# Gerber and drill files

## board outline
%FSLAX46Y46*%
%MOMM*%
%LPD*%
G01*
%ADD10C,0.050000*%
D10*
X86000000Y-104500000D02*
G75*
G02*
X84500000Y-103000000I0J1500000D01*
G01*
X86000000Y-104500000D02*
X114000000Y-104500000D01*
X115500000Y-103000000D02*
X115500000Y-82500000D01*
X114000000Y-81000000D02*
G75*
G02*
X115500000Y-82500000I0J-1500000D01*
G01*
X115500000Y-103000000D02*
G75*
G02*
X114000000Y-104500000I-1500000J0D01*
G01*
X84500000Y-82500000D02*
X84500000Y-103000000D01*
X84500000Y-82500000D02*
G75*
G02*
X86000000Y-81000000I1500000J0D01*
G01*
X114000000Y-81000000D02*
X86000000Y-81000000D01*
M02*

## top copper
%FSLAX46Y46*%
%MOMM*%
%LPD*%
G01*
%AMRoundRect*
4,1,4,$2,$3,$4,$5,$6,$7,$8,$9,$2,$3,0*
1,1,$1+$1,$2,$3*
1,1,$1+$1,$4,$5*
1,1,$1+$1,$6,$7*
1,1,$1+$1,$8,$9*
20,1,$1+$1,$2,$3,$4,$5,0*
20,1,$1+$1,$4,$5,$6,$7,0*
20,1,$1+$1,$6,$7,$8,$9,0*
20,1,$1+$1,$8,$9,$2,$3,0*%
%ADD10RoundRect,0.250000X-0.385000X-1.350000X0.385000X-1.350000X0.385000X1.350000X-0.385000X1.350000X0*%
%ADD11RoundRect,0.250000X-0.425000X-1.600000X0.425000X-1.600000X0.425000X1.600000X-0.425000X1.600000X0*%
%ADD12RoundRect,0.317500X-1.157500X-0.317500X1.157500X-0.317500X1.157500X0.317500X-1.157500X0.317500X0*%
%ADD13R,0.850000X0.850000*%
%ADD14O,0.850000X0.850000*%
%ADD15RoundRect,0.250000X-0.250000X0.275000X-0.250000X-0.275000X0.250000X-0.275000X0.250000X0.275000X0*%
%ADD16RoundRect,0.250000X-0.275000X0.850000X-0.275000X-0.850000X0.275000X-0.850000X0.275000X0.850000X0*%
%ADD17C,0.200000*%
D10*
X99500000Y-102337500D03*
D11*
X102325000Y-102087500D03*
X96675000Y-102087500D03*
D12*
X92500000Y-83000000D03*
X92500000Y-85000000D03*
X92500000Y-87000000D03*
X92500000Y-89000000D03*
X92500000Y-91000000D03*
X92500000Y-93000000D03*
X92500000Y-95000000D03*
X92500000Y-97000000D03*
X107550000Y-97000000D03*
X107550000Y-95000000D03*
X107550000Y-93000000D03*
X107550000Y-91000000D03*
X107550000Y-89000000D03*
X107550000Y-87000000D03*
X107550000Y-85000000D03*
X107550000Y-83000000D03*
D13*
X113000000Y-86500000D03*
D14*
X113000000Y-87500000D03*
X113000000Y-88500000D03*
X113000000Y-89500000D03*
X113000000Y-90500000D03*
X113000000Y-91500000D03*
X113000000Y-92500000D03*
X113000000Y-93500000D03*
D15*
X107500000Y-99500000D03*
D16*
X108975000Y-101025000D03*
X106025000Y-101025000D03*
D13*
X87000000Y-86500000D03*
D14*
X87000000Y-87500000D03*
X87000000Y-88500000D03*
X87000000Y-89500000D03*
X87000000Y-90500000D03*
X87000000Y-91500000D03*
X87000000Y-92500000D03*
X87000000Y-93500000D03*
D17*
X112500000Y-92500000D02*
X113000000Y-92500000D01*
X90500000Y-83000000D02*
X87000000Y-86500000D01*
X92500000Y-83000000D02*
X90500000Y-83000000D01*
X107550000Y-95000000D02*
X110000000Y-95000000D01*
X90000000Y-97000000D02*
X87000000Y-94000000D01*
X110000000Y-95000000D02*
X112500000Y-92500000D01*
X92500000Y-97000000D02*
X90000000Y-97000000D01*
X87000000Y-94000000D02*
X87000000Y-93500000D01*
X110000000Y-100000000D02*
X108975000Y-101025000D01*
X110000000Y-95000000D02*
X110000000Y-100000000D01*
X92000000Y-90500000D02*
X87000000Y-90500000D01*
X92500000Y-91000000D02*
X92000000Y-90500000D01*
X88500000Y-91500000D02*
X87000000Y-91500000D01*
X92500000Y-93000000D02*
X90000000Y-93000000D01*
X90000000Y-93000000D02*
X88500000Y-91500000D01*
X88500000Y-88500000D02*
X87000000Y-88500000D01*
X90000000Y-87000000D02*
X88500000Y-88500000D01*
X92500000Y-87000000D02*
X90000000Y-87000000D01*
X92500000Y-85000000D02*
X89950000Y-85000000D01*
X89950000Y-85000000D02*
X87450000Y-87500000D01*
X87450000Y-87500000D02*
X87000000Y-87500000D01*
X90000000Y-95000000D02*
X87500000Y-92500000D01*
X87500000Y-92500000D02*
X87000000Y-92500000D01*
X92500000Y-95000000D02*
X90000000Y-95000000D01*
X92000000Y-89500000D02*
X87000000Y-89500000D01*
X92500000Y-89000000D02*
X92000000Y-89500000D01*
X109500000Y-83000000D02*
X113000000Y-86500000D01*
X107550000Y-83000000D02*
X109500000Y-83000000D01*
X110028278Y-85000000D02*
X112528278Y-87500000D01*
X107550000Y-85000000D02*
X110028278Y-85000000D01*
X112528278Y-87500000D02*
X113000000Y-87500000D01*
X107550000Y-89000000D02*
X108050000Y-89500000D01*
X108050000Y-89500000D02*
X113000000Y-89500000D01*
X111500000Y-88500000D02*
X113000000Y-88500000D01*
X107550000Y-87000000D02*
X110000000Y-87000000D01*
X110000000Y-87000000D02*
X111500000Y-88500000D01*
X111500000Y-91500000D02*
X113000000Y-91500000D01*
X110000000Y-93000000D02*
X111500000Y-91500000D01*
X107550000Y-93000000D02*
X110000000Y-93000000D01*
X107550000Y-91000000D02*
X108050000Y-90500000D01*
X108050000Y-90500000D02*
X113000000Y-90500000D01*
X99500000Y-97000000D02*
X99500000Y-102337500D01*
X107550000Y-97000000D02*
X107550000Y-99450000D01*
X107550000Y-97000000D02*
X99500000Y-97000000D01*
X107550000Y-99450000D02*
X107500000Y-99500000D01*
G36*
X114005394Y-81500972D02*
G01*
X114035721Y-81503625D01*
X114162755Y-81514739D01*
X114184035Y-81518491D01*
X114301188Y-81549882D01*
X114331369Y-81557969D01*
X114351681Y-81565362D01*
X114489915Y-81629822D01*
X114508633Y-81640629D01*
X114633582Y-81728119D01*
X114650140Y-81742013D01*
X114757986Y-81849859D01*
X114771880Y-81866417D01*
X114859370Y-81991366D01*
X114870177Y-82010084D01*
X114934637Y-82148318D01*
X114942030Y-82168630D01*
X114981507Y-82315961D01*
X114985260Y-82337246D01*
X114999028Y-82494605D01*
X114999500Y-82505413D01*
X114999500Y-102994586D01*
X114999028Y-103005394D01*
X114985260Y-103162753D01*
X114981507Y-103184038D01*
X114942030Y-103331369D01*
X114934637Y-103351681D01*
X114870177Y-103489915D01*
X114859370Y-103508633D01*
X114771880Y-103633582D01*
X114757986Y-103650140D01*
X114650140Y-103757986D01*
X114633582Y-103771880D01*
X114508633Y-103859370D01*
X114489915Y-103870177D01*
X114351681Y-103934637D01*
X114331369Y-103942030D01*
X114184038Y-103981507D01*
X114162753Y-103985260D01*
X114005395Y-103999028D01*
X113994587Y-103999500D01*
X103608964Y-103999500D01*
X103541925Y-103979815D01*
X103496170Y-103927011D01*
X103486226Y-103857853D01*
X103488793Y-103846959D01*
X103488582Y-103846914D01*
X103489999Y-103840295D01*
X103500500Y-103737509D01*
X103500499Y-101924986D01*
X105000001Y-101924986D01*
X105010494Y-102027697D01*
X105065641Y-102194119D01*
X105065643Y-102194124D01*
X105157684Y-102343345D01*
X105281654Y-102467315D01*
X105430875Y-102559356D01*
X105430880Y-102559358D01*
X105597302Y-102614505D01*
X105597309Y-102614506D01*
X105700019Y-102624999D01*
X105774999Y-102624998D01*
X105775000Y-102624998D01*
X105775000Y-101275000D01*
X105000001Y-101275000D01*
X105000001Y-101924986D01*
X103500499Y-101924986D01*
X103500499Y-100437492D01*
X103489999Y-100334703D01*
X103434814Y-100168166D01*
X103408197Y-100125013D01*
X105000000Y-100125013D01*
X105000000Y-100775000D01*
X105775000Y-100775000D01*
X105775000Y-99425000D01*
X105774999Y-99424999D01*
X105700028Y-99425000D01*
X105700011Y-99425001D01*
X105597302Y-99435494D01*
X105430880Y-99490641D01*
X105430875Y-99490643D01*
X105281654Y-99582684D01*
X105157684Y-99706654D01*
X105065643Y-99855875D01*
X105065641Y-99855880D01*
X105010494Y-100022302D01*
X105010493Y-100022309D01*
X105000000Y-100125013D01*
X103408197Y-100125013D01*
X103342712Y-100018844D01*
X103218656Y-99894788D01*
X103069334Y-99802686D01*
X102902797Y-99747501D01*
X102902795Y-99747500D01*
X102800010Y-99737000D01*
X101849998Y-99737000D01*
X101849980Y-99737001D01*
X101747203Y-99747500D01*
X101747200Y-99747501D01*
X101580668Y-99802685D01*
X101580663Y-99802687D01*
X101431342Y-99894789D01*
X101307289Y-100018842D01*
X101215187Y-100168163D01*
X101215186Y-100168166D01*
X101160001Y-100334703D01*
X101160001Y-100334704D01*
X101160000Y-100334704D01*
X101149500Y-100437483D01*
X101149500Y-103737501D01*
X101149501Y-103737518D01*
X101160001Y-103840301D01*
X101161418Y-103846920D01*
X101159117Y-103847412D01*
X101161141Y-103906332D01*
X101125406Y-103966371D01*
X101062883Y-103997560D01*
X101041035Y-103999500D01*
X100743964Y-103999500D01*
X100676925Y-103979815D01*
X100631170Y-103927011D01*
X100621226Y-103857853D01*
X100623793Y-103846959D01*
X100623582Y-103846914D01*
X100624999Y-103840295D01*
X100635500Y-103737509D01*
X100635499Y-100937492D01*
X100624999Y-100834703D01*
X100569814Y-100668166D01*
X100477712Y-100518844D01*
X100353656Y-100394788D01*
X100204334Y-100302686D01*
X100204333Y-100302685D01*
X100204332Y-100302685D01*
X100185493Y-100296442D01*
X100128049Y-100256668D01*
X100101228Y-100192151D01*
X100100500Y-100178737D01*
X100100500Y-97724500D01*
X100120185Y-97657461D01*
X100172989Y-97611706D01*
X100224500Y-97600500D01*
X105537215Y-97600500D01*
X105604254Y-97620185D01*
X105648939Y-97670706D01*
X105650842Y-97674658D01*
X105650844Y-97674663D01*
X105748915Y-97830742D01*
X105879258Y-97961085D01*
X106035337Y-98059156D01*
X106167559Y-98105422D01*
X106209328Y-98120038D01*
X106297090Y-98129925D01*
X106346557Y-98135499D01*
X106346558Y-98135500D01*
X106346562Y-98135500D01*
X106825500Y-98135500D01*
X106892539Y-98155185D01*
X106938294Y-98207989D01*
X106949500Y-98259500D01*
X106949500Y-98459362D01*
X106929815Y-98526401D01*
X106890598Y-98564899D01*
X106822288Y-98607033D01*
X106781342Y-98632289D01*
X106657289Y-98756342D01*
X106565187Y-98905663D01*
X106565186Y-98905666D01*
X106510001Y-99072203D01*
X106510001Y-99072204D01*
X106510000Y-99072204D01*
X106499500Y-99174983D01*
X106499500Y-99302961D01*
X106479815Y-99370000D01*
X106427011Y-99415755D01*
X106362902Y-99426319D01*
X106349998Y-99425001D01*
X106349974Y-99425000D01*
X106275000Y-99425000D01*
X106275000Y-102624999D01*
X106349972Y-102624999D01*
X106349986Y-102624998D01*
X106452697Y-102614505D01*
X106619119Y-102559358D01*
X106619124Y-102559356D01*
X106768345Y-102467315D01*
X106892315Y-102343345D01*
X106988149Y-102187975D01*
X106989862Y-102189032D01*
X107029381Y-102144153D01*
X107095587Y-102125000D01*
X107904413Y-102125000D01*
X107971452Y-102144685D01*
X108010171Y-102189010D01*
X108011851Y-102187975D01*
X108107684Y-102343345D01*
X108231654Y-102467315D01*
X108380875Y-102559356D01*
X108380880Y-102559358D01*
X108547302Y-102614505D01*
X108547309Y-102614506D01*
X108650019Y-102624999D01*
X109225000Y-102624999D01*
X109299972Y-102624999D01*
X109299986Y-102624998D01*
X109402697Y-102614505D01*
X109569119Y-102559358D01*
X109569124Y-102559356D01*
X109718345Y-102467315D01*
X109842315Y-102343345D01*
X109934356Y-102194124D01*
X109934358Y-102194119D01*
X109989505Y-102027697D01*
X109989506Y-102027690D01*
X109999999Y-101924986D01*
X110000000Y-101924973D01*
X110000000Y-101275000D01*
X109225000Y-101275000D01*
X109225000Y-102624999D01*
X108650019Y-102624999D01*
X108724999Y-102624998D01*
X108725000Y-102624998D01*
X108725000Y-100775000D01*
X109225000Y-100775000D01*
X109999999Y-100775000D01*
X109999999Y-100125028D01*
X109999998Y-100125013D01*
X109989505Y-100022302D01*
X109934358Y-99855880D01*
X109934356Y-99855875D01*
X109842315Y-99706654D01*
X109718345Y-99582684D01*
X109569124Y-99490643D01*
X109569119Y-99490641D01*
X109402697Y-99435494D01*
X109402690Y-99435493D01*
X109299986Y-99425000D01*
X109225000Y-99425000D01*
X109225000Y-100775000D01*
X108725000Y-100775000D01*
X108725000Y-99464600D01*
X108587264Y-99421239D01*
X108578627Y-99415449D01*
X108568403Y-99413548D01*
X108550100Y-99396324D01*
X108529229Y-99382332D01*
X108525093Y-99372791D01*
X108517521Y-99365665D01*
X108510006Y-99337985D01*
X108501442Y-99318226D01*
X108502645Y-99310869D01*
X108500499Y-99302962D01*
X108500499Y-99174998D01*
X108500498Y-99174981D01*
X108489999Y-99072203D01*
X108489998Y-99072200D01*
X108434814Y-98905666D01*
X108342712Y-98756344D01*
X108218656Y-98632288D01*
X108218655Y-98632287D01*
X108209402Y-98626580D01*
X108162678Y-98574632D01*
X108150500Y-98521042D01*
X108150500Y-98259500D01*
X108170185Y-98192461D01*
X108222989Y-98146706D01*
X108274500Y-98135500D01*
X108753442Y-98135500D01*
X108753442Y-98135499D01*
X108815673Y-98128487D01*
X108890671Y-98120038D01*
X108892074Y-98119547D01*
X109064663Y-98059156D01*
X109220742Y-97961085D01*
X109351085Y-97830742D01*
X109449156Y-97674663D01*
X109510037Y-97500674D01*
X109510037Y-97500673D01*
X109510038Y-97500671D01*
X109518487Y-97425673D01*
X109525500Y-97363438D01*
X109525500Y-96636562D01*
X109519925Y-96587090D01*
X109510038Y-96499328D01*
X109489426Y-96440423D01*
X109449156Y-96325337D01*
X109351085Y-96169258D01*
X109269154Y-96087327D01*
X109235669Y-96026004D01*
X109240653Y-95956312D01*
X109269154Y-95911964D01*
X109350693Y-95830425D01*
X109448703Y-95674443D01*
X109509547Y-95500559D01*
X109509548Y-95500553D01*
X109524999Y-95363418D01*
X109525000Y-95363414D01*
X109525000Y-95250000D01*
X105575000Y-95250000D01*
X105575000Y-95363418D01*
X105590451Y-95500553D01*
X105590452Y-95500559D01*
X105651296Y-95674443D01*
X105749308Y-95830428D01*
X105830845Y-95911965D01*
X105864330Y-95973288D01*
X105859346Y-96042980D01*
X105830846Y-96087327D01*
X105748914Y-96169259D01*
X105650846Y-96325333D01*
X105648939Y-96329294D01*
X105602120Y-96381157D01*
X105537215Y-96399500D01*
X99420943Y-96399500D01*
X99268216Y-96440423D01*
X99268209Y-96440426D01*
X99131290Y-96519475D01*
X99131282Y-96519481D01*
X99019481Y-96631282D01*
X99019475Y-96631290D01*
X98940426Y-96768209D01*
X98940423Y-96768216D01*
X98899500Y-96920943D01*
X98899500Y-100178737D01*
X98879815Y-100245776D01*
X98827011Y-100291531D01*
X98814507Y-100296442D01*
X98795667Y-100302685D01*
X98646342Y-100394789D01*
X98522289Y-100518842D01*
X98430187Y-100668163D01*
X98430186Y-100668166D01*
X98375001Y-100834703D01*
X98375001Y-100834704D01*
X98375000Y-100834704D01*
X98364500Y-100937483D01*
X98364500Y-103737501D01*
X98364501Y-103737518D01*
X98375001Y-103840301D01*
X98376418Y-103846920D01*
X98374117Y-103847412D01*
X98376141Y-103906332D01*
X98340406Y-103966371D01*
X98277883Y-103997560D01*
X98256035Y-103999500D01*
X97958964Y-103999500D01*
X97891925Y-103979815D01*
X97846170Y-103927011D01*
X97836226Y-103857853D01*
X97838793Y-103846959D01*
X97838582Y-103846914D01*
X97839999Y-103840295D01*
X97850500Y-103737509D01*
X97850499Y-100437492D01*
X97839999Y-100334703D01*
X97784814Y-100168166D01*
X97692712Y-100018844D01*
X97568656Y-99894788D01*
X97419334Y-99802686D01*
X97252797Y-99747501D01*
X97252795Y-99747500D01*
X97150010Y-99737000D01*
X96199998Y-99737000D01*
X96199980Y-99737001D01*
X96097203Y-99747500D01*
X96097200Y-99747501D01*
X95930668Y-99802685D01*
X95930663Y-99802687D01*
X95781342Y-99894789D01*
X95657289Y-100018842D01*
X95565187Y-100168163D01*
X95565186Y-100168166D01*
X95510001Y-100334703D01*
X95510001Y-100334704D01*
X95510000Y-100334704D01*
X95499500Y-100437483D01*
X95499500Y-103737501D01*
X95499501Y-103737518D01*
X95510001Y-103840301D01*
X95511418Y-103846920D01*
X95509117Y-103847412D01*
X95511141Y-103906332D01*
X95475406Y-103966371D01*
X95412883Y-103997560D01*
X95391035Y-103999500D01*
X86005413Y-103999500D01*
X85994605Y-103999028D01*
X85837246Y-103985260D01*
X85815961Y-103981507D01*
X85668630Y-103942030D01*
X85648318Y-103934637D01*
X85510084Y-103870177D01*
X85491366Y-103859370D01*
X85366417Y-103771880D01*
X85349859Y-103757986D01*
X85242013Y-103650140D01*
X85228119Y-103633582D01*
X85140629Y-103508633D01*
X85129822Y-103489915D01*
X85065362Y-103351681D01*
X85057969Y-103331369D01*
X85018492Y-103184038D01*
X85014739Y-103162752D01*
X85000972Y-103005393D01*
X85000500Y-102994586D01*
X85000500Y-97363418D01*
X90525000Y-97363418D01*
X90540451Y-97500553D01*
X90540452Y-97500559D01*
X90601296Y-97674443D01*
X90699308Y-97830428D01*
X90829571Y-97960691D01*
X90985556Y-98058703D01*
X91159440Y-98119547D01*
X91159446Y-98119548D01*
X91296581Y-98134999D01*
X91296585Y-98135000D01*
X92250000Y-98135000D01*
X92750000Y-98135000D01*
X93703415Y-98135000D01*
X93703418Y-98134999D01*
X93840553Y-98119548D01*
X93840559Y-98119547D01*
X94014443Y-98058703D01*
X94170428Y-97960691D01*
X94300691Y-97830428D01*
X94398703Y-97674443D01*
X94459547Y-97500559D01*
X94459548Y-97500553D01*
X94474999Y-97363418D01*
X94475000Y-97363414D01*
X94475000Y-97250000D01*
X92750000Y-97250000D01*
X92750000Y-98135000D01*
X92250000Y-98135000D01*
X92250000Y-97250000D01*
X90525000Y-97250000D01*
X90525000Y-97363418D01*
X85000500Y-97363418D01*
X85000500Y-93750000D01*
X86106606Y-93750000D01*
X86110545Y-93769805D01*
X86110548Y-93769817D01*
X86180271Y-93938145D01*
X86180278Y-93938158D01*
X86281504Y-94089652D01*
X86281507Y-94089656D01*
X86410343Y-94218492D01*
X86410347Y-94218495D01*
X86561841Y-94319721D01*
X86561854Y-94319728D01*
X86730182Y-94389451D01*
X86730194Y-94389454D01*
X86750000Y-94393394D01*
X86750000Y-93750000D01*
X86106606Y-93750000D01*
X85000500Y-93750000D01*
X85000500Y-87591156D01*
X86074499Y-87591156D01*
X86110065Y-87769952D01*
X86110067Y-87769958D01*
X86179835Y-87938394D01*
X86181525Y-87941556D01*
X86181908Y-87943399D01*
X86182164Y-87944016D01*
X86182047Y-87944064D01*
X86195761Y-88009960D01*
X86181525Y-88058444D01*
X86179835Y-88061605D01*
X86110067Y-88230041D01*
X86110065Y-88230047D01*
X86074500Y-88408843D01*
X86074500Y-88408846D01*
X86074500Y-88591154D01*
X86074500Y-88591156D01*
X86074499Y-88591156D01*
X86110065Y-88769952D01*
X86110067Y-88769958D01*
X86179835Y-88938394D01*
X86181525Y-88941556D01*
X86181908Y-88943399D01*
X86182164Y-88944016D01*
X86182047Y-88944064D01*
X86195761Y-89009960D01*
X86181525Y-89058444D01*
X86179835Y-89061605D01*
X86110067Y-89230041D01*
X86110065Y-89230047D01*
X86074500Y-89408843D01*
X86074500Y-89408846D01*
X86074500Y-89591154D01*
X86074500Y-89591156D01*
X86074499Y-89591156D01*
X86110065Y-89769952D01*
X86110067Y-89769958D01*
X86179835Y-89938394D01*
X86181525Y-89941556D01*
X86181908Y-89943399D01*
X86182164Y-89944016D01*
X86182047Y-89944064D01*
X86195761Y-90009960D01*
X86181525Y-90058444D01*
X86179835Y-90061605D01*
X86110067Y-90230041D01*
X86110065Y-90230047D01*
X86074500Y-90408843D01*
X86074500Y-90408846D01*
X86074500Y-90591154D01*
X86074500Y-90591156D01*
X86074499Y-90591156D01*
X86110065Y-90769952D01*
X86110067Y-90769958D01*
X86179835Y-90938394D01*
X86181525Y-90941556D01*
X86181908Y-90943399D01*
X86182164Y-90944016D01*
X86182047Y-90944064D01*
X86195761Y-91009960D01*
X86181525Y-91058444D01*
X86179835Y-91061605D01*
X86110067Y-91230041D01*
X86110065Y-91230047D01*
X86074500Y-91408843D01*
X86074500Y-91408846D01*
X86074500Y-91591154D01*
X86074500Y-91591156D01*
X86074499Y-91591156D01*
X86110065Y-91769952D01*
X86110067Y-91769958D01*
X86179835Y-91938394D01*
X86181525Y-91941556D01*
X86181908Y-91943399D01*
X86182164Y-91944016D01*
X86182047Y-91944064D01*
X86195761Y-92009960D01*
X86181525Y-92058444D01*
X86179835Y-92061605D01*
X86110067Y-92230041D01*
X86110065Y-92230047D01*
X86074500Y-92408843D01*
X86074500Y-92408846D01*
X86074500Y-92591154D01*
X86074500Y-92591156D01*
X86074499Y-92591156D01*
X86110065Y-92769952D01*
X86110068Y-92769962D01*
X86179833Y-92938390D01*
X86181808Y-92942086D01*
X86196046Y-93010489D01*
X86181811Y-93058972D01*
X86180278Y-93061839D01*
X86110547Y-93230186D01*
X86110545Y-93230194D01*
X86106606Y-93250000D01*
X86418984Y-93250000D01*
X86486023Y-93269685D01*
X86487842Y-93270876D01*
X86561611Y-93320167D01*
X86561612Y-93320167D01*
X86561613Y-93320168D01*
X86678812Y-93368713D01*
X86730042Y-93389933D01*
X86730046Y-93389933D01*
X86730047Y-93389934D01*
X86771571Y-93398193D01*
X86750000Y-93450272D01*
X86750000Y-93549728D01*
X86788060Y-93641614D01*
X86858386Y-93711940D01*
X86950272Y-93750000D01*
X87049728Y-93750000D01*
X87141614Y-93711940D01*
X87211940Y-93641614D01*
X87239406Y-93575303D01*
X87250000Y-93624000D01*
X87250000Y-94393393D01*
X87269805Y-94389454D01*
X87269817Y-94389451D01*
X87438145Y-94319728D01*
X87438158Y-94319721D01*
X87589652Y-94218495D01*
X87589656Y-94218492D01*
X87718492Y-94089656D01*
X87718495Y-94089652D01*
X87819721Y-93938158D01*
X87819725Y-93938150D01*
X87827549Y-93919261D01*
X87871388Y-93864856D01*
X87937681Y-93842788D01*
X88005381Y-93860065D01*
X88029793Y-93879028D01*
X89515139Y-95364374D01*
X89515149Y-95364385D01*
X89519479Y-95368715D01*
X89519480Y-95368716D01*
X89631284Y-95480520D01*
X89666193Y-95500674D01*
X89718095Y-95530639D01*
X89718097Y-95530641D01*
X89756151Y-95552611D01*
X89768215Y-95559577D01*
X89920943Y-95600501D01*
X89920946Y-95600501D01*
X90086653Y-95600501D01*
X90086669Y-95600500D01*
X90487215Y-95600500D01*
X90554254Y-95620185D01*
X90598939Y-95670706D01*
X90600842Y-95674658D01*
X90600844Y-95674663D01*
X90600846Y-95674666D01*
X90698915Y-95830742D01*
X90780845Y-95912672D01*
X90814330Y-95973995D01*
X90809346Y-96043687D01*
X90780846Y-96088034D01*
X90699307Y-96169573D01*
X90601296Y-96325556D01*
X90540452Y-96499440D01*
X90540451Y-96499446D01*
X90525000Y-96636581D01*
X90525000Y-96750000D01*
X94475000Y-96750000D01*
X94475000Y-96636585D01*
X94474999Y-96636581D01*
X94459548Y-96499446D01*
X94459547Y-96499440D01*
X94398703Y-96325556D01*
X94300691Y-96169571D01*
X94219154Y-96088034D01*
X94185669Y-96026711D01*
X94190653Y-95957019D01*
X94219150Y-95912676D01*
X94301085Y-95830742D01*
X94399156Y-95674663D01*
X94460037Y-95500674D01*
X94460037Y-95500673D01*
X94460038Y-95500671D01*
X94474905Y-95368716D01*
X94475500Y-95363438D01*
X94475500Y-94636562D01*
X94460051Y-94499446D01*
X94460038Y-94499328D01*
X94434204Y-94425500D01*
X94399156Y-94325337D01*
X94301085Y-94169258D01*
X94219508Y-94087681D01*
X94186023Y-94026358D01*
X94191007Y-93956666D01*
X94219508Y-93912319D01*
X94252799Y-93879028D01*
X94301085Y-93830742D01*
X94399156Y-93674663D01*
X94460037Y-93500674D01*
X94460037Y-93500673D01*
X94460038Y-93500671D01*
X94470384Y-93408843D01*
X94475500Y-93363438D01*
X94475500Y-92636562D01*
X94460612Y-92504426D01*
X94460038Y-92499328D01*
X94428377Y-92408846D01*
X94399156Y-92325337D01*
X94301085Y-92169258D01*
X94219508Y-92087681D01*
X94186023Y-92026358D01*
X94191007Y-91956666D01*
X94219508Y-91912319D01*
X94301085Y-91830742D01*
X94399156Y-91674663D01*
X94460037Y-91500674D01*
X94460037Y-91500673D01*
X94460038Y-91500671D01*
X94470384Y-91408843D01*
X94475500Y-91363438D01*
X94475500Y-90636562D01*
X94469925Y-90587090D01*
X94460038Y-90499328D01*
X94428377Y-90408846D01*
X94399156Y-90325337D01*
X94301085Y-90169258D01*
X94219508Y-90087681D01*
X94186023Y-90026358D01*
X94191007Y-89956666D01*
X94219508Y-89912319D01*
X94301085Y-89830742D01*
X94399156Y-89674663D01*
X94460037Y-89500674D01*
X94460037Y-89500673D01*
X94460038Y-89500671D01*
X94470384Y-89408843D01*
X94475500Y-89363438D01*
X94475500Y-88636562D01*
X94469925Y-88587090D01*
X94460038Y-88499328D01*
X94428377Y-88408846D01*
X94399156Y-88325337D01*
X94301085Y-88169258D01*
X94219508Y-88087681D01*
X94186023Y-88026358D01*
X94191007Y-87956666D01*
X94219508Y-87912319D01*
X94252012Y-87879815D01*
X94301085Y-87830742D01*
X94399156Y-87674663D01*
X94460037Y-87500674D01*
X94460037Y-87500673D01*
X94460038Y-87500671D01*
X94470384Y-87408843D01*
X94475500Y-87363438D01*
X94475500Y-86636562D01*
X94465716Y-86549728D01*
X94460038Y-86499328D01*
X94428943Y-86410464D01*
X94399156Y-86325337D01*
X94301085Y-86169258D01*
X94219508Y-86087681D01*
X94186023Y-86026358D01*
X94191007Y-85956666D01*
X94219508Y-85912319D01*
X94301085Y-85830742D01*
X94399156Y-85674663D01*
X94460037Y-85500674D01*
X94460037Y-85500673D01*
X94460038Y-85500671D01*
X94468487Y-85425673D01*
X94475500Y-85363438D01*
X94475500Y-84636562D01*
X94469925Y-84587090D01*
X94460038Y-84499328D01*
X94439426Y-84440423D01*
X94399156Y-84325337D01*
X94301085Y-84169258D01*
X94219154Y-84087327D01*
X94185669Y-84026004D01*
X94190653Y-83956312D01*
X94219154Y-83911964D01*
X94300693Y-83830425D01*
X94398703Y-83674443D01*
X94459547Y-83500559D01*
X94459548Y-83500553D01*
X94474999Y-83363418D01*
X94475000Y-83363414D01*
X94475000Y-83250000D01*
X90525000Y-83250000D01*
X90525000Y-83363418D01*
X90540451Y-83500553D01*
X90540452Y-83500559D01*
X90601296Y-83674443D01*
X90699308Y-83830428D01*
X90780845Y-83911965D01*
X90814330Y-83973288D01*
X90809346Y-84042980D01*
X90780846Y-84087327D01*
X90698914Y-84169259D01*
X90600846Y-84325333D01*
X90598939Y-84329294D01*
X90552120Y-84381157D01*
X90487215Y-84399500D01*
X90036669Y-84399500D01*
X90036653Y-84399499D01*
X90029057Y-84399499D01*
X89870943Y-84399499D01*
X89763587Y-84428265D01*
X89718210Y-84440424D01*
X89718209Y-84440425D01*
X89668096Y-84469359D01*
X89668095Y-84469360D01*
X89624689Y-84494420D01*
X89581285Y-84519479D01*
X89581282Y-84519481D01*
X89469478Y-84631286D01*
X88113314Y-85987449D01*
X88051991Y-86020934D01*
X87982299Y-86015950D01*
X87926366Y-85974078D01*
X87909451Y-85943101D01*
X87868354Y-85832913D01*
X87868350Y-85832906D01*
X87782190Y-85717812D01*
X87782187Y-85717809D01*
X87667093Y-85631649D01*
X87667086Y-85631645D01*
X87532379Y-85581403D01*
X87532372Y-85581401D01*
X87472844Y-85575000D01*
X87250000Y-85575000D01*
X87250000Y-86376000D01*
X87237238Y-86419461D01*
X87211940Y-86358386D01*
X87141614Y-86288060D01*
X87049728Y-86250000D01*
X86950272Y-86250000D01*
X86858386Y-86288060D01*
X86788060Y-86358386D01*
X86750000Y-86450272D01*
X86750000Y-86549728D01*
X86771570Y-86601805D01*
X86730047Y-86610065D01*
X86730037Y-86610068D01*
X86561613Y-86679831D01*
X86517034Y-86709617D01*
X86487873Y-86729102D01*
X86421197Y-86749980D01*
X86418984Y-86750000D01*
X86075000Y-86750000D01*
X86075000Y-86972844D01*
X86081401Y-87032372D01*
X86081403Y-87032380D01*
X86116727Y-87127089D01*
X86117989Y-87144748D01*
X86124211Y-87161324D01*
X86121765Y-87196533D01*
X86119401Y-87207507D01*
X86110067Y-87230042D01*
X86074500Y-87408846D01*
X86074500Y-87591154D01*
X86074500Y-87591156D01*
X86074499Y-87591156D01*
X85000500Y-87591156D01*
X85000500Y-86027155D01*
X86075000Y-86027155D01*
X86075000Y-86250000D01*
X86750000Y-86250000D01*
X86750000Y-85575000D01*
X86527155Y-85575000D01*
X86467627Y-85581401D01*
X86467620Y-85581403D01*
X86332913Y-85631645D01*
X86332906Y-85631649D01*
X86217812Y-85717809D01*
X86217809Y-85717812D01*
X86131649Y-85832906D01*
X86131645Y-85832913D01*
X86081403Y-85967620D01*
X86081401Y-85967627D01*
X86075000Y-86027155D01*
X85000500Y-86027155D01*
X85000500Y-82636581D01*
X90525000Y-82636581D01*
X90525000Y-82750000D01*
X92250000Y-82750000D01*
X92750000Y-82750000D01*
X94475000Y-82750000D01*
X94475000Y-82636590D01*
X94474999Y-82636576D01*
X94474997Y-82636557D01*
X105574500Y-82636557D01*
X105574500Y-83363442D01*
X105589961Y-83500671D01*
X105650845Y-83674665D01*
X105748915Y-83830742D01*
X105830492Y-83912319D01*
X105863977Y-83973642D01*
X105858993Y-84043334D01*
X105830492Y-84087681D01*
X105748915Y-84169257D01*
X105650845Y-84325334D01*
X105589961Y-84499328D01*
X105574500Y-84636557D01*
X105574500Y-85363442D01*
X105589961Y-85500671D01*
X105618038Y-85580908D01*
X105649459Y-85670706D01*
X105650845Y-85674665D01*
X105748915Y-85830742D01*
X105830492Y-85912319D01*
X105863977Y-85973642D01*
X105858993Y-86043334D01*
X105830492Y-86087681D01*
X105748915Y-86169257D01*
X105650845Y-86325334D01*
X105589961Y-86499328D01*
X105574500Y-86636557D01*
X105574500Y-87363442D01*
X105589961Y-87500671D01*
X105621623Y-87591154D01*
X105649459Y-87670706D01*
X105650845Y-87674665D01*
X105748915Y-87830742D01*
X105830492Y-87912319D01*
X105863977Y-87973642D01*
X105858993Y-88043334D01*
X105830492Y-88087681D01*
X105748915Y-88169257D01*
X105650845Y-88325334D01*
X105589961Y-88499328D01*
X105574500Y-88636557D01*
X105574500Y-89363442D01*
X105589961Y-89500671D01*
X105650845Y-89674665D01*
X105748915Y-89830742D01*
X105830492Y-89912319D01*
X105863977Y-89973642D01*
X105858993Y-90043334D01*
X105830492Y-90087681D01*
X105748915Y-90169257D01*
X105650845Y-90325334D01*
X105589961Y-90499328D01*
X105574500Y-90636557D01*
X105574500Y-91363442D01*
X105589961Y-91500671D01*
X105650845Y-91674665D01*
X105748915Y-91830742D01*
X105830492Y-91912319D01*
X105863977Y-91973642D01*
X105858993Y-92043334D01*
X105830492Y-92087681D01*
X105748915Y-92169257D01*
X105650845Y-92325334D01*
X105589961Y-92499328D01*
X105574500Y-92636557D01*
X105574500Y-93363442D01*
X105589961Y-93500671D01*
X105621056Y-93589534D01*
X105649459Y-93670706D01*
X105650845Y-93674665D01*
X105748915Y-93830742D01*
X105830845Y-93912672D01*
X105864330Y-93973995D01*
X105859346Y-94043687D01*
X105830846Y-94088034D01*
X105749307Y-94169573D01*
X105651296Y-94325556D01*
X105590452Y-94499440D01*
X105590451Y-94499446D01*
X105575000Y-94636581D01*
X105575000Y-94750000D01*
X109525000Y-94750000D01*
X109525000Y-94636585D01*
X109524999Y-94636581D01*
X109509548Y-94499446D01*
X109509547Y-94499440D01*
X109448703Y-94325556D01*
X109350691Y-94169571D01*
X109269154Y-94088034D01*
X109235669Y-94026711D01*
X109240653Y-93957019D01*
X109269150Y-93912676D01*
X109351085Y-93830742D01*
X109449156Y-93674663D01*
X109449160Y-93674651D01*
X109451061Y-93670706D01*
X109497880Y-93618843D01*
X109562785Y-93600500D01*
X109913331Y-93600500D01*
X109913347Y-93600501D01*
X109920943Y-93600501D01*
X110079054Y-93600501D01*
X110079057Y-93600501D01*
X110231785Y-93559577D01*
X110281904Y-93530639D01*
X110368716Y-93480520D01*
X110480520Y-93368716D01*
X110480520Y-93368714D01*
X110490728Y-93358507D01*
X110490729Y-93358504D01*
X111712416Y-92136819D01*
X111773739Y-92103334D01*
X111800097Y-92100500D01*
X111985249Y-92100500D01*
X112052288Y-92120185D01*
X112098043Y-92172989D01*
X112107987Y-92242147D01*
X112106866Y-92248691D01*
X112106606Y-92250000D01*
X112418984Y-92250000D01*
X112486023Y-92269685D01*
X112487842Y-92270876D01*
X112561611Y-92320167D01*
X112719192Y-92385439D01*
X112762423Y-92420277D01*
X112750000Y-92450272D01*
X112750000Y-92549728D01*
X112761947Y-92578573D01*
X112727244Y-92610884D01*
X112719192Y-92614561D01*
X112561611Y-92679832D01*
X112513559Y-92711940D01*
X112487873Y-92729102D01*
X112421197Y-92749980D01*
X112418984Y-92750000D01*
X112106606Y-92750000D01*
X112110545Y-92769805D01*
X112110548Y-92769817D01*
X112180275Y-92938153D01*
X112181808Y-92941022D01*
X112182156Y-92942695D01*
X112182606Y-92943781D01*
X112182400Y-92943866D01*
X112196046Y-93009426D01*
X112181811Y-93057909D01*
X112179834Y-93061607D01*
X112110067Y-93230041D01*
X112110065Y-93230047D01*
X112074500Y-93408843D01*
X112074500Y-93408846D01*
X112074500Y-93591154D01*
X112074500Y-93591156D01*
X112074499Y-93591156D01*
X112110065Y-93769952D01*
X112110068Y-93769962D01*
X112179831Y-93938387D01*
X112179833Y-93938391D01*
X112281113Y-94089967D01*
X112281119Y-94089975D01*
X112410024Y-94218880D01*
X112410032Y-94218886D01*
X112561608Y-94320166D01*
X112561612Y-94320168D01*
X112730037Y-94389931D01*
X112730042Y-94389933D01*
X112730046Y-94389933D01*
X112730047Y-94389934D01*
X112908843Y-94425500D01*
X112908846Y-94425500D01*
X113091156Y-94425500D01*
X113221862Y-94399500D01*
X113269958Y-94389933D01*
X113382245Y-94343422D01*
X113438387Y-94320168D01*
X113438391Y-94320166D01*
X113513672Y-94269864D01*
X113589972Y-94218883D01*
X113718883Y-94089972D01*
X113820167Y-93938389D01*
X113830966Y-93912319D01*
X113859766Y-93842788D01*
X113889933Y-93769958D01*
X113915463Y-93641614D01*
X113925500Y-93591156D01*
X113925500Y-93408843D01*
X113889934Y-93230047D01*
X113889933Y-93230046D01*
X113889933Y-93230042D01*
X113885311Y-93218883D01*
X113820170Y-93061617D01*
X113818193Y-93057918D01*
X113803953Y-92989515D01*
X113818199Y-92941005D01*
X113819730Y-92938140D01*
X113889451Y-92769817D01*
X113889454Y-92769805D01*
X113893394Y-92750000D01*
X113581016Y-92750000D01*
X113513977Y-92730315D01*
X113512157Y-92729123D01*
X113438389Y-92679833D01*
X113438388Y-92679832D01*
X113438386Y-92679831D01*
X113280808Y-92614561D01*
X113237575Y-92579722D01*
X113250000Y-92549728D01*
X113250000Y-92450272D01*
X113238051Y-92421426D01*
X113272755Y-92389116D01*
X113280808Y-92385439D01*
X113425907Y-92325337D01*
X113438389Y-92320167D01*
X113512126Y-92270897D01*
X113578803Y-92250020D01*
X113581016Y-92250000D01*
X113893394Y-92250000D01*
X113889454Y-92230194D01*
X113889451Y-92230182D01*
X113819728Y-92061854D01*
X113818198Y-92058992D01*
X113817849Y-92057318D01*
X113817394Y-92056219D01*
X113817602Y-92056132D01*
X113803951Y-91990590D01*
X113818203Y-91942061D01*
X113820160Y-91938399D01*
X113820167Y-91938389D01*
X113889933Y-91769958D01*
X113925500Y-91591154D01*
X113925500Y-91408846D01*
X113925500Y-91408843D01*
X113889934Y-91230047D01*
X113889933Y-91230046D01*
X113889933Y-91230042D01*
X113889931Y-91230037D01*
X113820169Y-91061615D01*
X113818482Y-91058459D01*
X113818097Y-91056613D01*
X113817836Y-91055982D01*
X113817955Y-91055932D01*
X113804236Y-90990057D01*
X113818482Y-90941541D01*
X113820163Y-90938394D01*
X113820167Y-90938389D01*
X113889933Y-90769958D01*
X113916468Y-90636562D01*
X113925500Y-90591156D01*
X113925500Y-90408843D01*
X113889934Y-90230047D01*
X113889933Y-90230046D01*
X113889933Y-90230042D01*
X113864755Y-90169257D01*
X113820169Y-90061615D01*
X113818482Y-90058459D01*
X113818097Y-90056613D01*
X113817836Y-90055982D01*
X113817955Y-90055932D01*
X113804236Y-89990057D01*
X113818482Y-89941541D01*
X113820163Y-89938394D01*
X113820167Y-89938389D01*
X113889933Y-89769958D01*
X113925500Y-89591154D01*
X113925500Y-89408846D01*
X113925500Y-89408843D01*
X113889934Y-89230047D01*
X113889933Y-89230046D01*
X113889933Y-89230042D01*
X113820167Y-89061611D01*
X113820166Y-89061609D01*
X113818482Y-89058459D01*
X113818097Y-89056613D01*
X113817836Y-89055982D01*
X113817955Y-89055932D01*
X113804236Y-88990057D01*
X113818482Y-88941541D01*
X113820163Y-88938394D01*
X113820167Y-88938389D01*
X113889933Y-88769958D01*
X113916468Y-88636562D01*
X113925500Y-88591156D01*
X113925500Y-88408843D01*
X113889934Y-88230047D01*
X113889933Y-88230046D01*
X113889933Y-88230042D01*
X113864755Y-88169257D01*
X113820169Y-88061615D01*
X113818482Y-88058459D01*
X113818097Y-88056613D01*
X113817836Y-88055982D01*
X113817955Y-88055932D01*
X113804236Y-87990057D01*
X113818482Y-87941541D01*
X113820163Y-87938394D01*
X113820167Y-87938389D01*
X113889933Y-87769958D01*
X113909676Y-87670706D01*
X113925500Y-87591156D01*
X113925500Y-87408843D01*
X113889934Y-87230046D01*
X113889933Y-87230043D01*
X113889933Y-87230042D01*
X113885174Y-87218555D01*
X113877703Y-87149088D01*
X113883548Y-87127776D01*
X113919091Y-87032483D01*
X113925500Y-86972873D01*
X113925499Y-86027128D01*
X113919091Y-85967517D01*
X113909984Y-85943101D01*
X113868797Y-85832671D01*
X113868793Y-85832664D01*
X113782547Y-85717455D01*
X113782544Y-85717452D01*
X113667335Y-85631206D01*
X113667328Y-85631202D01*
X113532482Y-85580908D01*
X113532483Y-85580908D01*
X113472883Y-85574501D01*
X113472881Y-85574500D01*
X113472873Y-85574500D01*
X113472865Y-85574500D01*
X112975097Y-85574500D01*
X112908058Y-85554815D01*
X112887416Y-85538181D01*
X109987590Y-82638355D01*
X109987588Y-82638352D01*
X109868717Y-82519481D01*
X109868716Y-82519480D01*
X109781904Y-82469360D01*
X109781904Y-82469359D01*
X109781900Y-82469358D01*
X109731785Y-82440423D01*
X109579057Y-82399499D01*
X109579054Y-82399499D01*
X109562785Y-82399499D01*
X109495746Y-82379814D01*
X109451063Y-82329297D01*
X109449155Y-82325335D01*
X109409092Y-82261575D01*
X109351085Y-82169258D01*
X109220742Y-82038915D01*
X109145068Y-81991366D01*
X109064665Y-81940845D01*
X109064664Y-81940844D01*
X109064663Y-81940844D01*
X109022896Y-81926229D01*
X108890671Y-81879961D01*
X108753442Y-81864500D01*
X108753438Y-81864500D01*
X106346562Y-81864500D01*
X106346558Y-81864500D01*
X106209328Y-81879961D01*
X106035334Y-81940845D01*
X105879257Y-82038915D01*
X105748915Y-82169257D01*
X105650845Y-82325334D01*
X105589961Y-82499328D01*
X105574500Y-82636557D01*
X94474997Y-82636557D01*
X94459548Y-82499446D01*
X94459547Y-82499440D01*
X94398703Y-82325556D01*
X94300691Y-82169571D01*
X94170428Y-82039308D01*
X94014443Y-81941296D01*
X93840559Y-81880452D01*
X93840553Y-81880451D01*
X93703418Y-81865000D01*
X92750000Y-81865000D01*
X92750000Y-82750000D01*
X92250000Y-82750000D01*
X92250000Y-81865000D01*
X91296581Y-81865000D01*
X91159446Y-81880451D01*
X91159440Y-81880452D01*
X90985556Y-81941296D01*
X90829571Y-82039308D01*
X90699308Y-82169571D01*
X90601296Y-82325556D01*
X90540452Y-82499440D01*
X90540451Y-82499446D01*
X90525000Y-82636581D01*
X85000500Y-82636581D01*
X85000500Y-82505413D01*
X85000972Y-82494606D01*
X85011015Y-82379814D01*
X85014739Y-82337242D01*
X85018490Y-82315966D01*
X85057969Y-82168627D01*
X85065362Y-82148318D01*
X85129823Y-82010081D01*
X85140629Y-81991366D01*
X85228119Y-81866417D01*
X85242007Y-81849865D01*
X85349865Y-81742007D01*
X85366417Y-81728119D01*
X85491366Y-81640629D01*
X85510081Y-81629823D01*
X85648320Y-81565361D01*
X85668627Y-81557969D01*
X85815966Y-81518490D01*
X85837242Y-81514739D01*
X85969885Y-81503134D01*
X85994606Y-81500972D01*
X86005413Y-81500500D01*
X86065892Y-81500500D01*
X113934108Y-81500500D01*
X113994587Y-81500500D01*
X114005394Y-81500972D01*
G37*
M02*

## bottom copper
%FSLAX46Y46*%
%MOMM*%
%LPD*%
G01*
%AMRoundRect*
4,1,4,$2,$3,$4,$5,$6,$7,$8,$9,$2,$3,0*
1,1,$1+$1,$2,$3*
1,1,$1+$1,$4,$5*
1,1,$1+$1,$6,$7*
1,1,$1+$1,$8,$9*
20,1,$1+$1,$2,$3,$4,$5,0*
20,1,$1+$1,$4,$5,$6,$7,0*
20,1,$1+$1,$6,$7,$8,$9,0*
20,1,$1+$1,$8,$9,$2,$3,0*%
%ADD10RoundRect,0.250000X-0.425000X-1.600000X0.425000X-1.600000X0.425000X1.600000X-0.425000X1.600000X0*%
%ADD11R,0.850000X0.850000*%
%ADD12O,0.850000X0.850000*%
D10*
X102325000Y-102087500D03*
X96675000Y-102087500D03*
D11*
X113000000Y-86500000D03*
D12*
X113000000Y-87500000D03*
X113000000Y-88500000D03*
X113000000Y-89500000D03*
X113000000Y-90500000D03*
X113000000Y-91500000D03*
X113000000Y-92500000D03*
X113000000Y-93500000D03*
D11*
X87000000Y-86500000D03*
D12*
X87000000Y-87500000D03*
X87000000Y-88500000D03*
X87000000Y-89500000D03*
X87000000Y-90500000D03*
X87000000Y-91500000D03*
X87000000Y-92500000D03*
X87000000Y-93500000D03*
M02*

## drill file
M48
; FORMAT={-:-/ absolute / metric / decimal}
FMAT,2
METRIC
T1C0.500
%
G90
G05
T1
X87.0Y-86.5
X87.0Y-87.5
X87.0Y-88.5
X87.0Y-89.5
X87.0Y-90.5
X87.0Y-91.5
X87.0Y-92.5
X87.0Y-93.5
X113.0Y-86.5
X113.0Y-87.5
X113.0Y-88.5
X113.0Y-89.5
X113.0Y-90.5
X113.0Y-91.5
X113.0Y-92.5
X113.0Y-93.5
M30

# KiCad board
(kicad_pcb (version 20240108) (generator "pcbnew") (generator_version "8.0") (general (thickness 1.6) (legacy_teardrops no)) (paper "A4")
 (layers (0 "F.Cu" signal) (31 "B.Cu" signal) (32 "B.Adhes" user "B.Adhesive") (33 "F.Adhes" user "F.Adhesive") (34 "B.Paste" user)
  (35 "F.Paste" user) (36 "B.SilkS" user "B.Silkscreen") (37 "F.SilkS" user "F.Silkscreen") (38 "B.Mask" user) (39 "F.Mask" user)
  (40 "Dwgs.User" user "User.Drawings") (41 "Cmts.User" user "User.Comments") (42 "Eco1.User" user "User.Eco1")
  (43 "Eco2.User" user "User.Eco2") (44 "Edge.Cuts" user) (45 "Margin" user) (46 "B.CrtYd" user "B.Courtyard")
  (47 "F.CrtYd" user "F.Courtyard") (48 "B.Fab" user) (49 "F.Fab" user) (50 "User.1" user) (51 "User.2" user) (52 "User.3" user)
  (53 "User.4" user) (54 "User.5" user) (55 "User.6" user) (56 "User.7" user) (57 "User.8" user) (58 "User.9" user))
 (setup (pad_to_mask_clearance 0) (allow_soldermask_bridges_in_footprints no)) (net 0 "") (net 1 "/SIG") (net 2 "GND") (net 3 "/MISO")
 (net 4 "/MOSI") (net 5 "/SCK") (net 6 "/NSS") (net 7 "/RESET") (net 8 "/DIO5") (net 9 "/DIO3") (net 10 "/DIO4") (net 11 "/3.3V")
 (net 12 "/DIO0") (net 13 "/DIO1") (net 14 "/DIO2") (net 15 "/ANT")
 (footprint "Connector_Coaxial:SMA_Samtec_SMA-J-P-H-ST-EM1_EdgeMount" (layer "F.Cu") (at 99.5 102.3375 -90)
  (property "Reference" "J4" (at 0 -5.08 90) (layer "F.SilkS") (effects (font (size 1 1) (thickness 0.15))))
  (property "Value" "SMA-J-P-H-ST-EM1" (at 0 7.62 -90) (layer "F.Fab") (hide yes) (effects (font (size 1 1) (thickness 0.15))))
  (pad "1" smd roundrect (at 0 0) (size 1.27 3.2) (layers "F.Cu" "F.Mask") (roundrect_rratio 0.1968503937) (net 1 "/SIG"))
  (pad "2" smd roundrect (at -0.25 -2.825) (size 1.35 3.7) (layers "F.Cu" "F.Mask") (roundrect_rratio 0.1851851852))
  (pad "2" smd roundrect (at -0.25 -2.825) (size 1.35 3.7) (layers "B.Cu" "B.Mask") (roundrect_rratio 0.1851851852))
  (pad "2" smd roundrect (at -0.25 2.825) (size 1.35 3.7) (layers "F.Cu" "F.Mask") (roundrect_rratio 0.1851851852))
  (pad "2" smd roundrect (at -0.25 2.825) (size 1.35 3.7) (layers "B.Cu" "B.Mask") (roundrect_rratio 0.1851851852)))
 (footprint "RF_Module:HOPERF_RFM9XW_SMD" (layer "F.Cu") (at 100.025 90)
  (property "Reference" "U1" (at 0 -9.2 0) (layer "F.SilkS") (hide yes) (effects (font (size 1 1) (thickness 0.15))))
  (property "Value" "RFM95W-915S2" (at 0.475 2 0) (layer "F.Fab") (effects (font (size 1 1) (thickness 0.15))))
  (pad "1" smd roundrect (at -7.525 -7) (size 2.95 1.27) (layers "F.Cu" "F.Paste" "F.Mask") (roundrect_rratio 0.25) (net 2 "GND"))
  (pad "2" smd roundrect (at -7.525 -5) (size 2.95 1.27) (layers "F.Cu" "F.Paste" "F.Mask") (roundrect_rratio 0.25) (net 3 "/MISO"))
  (pad "3" smd roundrect (at -7.525 -3) (size 2.95 1.27) (layers "F.Cu" "F.Paste" "F.Mask") (roundrect_rratio 0.25) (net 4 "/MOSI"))
  (pad "4" smd roundrect (at -7.525 -1) (size 2.95 1.27) (layers "F.Cu" "F.Paste" "F.Mask") (roundrect_rratio 0.25) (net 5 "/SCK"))
  (pad "5" smd roundrect (at -7.525 1) (size 2.95 1.27) (layers "F.Cu" "F.Paste" "F.Mask") (roundrect_rratio 0.25) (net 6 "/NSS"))
  (pad "6" smd roundrect (at -7.525 3) (size 2.95 1.27) (layers "F.Cu" "F.Paste" "F.Mask") (roundrect_rratio 0.25) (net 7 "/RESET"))
  (pad "7" smd roundrect (at -7.525 5) (size 2.95 1.27) (layers "F.Cu" "F.Paste" "F.Mask") (roundrect_rratio 0.25) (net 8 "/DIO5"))
  (pad "8" smd roundrect (at -7.525 7) (size 2.95 1.27) (layers "F.Cu" "F.Paste" "F.Mask") (roundrect_rratio 0.25) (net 2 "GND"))
  (pad "9" smd roundrect (at 7.525 7) (size 2.95 1.27) (layers "F.Cu" "F.Paste" "F.Mask") (roundrect_rratio 0.25) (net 1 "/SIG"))
  (pad "10" smd roundrect (at 7.525 5) (size 2.95 1.27) (layers "F.Cu" "F.Paste" "F.Mask") (roundrect_rratio 0.25) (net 2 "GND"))
  (pad "11" smd roundrect (at 7.525 3) (size 2.95 1.27) (layers "F.Cu" "F.Paste" "F.Mask") (roundrect_rratio 0.25) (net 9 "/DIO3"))
  (pad "12" smd roundrect (at 7.525 1) (size 2.95 1.27) (layers "F.Cu" "F.Paste" "F.Mask") (roundrect_rratio 0.25) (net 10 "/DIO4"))
  (pad "13" smd roundrect (at 7.525 -1) (size 2.95 1.27) (layers "F.Cu" "F.Paste" "F.Mask") (roundrect_rratio 0.25) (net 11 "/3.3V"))
  (pad "14" smd roundrect (at 7.525 -3) (size 2.95 1.27) (layers "F.Cu" "F.Paste" "F.Mask") (roundrect_rratio 0.25) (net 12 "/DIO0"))
  (pad "15" smd roundrect (at 7.525 -5) (size 2.95 1.27) (layers "F.Cu" "F.Paste" "F.Mask") (roundrect_rratio 0.25) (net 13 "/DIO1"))
  (pad "16" smd roundrect (at 7.525 -7) (size 2.95 1.27) (layers "F.Cu" "F.Paste" "F.Mask") (roundrect_rratio 0.25) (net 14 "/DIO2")))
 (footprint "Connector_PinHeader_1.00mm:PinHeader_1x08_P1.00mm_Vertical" (layer "F.Cu") (at 113 86.5)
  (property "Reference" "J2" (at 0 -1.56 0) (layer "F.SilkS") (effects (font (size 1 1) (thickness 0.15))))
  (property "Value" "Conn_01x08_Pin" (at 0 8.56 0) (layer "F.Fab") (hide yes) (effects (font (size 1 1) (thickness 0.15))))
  (pad "1" thru_hole rect (at 0 0) (size 0.85 0.85) (drill 0.5) (layers "*.Cu" "*.Mask") (remove_unused_layers no) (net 14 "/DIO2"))
  (pad "2" thru_hole oval (at 0 1) (size 0.85 0.85) (drill 0.5) (layers "*.Cu" "*.Mask") (remove_unused_layers no) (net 13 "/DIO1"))
  (pad "3" thru_hole oval (at 0 2) (size 0.85 0.85) (drill 0.5) (layers "*.Cu" "*.Mask") (remove_unused_layers no) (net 12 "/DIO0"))
  (pad "4" thru_hole oval (at 0 3) (size 0.85 0.85) (drill 0.5) (layers "*.Cu" "*.Mask") (remove_unused_layers no) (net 11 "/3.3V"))
  (pad "5" thru_hole oval (at 0 4) (size 0.85 0.85) (drill 0.5) (layers "*.Cu" "*.Mask") (remove_unused_layers no) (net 10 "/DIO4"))
  (pad "6" thru_hole oval (at 0 5) (size 0.85 0.85) (drill 0.5) (layers "*.Cu" "*.Mask") (remove_unused_layers no) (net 9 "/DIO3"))
  (pad "7" thru_hole oval (at 0 6) (size 0.85 0.85) (drill 0.5) (layers "*.Cu" "*.Mask") (remove_unused_layers no) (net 2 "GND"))
  (pad "8" thru_hole oval (at 0 7) (size 0.85 0.85) (drill 0.5) (layers "*.Cu" "*.Mask") (remove_unused_layers no) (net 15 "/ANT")))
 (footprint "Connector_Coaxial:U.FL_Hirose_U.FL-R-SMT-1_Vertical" (layer "F.Cu") (at 107.5 100.55 -90)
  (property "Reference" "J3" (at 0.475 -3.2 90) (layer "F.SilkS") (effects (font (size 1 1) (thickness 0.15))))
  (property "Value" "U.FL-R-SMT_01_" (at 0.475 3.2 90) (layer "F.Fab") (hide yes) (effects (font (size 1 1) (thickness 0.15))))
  (pad "1" smd roundrect (at -1.05 0 270) (size 1.05 1) (layers "F.Cu" "F.Paste" "F.Mask") (roundrect_rratio 0.25) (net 1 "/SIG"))
  (pad "2" smd roundrect (at 0.475 -1.475 270) (size 2.2 1.05) (layers "F.Cu" "F.Paste" "F.Mask") (roundrect_rratio 0.2380952381)
   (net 2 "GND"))
  (pad "2" smd roundrect (at 0.475 1.475 270) (size 2.2 1.05) (layers "F.Cu" "F.Paste" "F.Mask") (roundrect_rratio 0.2380952381)
   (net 2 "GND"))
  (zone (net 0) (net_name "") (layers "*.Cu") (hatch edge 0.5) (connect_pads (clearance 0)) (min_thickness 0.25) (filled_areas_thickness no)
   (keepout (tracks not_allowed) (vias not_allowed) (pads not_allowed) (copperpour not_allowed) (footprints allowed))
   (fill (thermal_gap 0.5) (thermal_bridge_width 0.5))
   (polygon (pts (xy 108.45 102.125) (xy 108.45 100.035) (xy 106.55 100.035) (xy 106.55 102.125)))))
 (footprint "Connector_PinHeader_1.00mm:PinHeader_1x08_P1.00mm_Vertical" (layer "F.Cu") (at 87 86.5)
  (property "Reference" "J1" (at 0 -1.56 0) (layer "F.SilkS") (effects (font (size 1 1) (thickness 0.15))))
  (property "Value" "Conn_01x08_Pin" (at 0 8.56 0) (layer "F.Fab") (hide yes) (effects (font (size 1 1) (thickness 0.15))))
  (pad "1" thru_hole rect (at 0 0) (size 0.85 0.85) (drill 0.5) (layers "*.Cu" "*.Mask") (remove_unused_layers no) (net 2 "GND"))
  (pad "2" thru_hole oval (at 0 1) (size 0.85 0.85) (drill 0.5) (layers "*.Cu" "*.Mask") (remove_unused_layers no) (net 3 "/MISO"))
  (pad "3" thru_hole oval (at 0 2) (size 0.85 0.85) (drill 0.5) (layers "*.Cu" "*.Mask") (remove_unused_layers no) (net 4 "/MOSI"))
  (pad "4" thru_hole oval (at 0 3) (size 0.85 0.85) (drill 0.5) (layers "*.Cu" "*.Mask") (remove_unused_layers no) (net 5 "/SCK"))
  (pad "5" thru_hole oval (at 0 4) (size 0.85 0.85) (drill 0.5) (layers "*.Cu" "*.Mask") (remove_unused_layers no) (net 6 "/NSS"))
  (pad "6" thru_hole oval (at 0 5) (size 0.85 0.85) (drill 0.5) (layers "*.Cu" "*.Mask") (remove_unused_layers no) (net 7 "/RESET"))
  (pad "7" thru_hole oval (at 0 6) (size 0.85 0.85) (drill 0.5) (layers "*.Cu" "*.Mask") (remove_unused_layers no) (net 8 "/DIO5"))
  (pad "8" thru_hole oval (at 0 7) (size 0.85 0.85) (drill 0.5) (layers "*.Cu" "*.Mask") (remove_unused_layers no) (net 2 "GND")))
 (gr_arc (start 86 104.5) (mid 84.93934 104.06066) (end 84.5 103) (stroke (width 0.05) (type default)) (layer "Edge.Cuts"))
 (gr_line (start 86 104.5) (end 114 104.5) (stroke (width 0.05) (type default)) (layer "Edge.Cuts"))
 (gr_line (start 115.5 103) (end 115.5 82.5) (stroke (width 0.05) (type default)) (layer "Edge.Cuts"))
 (gr_arc (start 114 81) (mid 115.06066 81.43934) (end 115.5 82.5) (stroke (width 0.05) (type default)) (layer "Edge.Cuts"))
 (gr_arc (start 115.5 103) (mid 115.06066 104.06066) (end 114 104.5) (stroke (width 0.05) (type default)) (layer "Edge.Cuts"))
 (gr_line (start 84.5 82.5) (end 84.5 103) (stroke (width 0.05) (type default)) (layer "Edge.Cuts"))
 (gr_arc (start 84.5 82.5) (mid 84.93934 81.43934) (end 86 81) (stroke (width 0.05) (type default)) (layer "Edge.Cuts"))
 (gr_line (start 114 81) (end 86 81) (stroke (width 0.05) (type default)) (layer "Edge.Cuts"))
 (segment (start 112.5 92.5) (end 113 92.5) (width 0.2) (layer "F.Cu") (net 2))
 (segment (start 90.5 83) (end 87 86.5) (width 0.2) (layer "F.Cu") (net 2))
 (segment (start 92.5 83) (end 90.5 83) (width 0.2) (layer "F.Cu") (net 2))
 (segment (start 107.55 95) (end 110 95) (width 0.2) (layer "F.Cu") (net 2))
 (segment (start 90 97) (end 87 94) (width 0.2) (layer "F.Cu") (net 2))
 (segment (start 110 95) (end 112.5 92.5) (width 0.2) (layer "F.Cu") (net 2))
 (segment (start 92.5 97) (end 90 97) (width 0.2) (layer "F.Cu") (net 2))
 (segment (start 87 94) (end 87 93.5) (width 0.2) (layer "F.Cu") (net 2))
 (segment (start 110 100) (end 108.975 101.025) (width 0.2) (layer "F.Cu") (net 2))
 (segment (start 110 95) (end 110 100) (width 0.2) (layer "F.Cu") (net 2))
 (segment (start 92 90.5) (end 87 90.5) (width 0.2) (layer "F.Cu") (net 6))
 (segment (start 92.5 91) (end 92 90.5) (width 0.2) (layer "F.Cu") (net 6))
 (segment (start 88.5 91.5) (end 87 91.5) (width 0.2) (layer "F.Cu") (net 7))
 (segment (start 92.5 93) (end 90 93) (width 0.2) (layer "F.Cu") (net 7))
 (segment (start 90 93) (end 88.5 91.5) (width 0.2) (layer "F.Cu") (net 7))
 (segment (start 88.5 88.5) (end 87 88.5) (width 0.2) (layer "F.Cu") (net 4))
 (segment (start 90 87) (end 88.5 88.5) (width 0.2) (layer "F.Cu") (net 4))
 (segment (start 92.5 87) (end 90 87) (width 0.2) (layer "F.Cu") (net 4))
 (segment (start 92.5 85) (end 89.95 85) (width 0.2) (layer "F.Cu") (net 3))
 (segment (start 89.95 85) (end 87.45 87.5) (width 0.2) (layer "F.Cu") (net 3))
 (segment (start 87.45 87.5) (end 87 87.5) (width 0.2) (layer "F.Cu") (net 3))
 (segment (start 90 95) (end 87.5 92.5) (width 0.2) (layer "F.Cu") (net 8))
 (segment (start 87.5 92.5) (end 87 92.5) (width 0.2) (layer "F.Cu") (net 8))
 (segment (start 92.5 95) (end 90 95) (width 0.2) (layer "F.Cu") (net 8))
 (segment (start 92 89.5) (end 87 89.5) (width 0.2) (layer "F.Cu") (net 5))
 (segment (start 92.5 89) (end 92 89.5) (width 0.2) (layer "F.Cu") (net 5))
 (segment (start 109.5 83) (end 113 86.5) (width 0.2) (layer "F.Cu") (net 14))
 (segment (start 107.55 83) (end 109.5 83) (width 0.2) (layer "F.Cu") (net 14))
 (segment (start 110.028278 85) (end 112.528278 87.5) (width 0.2) (layer "F.Cu") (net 13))
 (segment (start 107.55 85) (end 110.028278 85) (width 0.2) (layer "F.Cu") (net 13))
 (segment (start 112.528278 87.5) (end 113 87.5) (width 0.2) (layer "F.Cu") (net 13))
 (segment (start 107.55 89) (end 108.05 89.5) (width 0.2) (layer "F.Cu") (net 11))
 (segment (start 108.05 89.5) (end 113 89.5) (width 0.2) (layer "F.Cu") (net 11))
 (segment (start 111.5 88.5) (end 113 88.5) (width 0.2) (layer "F.Cu") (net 12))
 (segment (start 107.55 87) (end 110 87) (width 0.2) (layer "F.Cu") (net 12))
 (segment (start 110 87) (end 111.5 88.5) (width 0.2) (layer "F.Cu") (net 12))
 (segment (start 111.5 91.5) (end 113 91.5) (width 0.2) (layer "F.Cu") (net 9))
 (segment (start 110 93) (end 111.5 91.5) (width 0.2) (layer "F.Cu") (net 9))
 (segment (start 107.55 93) (end 110 93) (width 0.2) (layer "F.Cu") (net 9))
 (segment (start 107.55 91) (end 108.05 90.5) (width 0.2) (layer "F.Cu") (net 10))
 (segment (start 108.05 90.5) (end 113 90.5) (width 0.2) (layer "F.Cu") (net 10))
 (segment (start 99.5 97) (end 99.5 102.3375) (width 0.2) (layer "F.Cu") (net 1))
 (segment (start 107.55 97) (end 107.55 99.45) (width 0.2) (layer "F.Cu") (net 1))
 (segment (start 107.55 97) (end 99.5 97) (width 0.2) (layer "F.Cu") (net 1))
 (segment (start 107.55 99.45) (end 107.5 99.5) (width 0.2) (layer "F.Cu") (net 1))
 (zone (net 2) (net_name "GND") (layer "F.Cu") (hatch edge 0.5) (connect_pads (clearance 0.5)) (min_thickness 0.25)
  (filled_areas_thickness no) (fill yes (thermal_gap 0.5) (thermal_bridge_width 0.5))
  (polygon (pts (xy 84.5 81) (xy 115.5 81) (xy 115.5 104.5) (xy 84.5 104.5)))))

